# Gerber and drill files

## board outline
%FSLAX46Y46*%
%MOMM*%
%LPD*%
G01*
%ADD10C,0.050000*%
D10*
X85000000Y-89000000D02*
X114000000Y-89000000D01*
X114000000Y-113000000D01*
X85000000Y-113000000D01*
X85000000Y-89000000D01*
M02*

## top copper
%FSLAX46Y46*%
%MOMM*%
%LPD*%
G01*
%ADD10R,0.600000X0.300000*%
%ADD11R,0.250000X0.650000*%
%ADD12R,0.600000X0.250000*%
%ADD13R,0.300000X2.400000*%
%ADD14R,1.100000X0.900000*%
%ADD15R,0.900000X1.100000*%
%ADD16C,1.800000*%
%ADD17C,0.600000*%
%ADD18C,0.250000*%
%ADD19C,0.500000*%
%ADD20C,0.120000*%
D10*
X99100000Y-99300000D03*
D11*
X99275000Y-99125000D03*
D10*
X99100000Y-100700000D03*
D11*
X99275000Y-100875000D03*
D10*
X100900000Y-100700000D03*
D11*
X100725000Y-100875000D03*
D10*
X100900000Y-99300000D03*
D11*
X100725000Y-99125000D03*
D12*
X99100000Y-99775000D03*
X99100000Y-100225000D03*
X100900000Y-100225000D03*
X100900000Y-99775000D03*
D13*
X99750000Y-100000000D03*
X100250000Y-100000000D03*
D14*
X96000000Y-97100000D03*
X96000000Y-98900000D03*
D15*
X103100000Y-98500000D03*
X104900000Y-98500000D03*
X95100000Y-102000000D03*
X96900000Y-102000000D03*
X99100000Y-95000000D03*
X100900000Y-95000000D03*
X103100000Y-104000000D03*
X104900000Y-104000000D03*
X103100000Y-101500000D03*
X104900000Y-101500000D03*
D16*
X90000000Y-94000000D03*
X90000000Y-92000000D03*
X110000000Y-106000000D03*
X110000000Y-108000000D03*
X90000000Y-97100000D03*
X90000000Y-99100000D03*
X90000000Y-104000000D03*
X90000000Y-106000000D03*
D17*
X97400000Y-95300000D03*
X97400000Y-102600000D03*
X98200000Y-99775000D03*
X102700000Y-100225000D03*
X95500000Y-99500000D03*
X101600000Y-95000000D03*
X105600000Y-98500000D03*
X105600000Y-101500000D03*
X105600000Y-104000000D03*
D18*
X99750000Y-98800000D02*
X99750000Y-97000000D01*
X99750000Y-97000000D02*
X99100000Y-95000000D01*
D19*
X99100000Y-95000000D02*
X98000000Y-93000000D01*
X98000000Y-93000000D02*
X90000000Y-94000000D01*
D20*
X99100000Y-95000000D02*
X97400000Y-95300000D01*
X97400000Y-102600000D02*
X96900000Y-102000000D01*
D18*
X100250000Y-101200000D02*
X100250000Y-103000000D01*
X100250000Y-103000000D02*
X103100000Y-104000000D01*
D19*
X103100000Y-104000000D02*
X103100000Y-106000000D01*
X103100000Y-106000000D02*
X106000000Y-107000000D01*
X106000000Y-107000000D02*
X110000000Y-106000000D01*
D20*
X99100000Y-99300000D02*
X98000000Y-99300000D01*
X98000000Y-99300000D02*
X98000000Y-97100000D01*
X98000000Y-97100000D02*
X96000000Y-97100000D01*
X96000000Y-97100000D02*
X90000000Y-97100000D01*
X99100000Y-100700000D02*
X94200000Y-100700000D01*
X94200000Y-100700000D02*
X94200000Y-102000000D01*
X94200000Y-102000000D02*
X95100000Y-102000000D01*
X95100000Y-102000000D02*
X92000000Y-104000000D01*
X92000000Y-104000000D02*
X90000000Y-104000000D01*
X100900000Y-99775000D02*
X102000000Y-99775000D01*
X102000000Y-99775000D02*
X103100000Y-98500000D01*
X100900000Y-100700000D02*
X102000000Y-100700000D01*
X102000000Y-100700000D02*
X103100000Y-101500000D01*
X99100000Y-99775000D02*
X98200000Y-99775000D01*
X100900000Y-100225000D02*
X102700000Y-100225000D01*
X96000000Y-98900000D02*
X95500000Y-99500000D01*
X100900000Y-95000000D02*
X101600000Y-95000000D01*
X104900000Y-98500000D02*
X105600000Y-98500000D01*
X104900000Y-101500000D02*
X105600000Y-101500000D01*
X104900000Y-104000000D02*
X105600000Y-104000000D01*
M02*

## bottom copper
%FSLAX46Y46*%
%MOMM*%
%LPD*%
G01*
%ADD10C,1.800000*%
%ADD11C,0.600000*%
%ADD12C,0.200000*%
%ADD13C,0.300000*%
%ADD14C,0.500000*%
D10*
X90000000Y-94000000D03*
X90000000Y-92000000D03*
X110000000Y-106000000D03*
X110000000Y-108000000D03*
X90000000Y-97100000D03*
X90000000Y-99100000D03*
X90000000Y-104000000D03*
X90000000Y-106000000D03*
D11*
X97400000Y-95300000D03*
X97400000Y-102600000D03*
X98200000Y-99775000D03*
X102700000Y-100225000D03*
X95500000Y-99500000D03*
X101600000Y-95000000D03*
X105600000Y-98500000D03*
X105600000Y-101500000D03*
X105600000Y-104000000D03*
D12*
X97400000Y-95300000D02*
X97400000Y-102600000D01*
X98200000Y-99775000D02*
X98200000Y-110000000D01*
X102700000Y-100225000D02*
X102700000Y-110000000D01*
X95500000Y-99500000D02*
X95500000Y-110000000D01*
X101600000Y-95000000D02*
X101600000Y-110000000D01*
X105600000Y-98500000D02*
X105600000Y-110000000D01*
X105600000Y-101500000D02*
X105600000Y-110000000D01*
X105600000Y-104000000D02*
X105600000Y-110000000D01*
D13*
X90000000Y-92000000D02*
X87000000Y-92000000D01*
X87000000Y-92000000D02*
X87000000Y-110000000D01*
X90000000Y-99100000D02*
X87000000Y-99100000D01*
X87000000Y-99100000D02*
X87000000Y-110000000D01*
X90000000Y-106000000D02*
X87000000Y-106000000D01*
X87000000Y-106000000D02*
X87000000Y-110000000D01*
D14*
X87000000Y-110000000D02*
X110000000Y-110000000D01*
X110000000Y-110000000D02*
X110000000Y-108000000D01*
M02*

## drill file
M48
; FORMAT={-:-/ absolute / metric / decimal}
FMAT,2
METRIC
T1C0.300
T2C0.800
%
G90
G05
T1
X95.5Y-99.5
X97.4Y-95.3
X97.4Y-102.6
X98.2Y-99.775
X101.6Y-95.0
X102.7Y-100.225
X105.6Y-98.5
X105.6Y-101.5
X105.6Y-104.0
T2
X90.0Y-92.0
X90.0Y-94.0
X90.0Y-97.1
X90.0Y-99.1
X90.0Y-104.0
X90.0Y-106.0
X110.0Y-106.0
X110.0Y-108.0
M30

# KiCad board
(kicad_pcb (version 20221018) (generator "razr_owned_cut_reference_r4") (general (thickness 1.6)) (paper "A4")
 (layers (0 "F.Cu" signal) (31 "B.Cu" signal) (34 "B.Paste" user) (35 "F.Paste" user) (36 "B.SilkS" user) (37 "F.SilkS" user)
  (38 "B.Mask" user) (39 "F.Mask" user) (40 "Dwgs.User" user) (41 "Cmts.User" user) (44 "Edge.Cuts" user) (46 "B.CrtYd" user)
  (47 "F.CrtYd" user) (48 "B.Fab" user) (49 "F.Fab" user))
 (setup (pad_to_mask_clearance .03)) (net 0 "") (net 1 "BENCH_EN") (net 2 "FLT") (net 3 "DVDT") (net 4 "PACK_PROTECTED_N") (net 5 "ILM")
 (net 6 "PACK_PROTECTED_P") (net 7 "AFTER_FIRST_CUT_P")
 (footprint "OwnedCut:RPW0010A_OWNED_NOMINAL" (layer "F.Cu") (at 100 100)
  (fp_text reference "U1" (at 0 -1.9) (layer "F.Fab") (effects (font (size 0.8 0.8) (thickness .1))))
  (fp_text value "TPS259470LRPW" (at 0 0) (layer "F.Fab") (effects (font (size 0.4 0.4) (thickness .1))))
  (pad "1" smd rect (at -0.9 -0.7) (size 0.6 0.3) (layers "F.Cu" "F.Paste" "F.Mask") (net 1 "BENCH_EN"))
  (pad "1" smd rect (at -0.725 -0.875) (size 0.25 0.65) (layers "F.Cu" "F.Paste" "F.Mask") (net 1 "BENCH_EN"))
  (pad "4" smd rect (at -0.9 0.7) (size 0.6 0.3) (layers "F.Cu" "F.Paste" "F.Mask") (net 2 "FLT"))
  (pad "4" smd rect (at -0.725 0.875) (size 0.25 0.65) (layers "F.Cu" "F.Paste" "F.Mask") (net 2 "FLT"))
  (pad "7" smd rect (at 0.9 0.7) (size 0.6 0.3) (layers "F.Cu" "F.Paste" "F.Mask") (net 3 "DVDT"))
  (pad "7" smd rect (at 0.725 0.875) (size 0.25 0.65) (layers "F.Cu" "F.Paste" "F.Mask") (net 3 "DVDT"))
  (pad "10" smd rect (at 0.9 -0.7) (size 0.6 0.3) (layers "F.Cu" "F.Paste" "F.Mask"))
  (pad "10" smd rect (at 0.725 -0.875) (size 0.25 0.65) (layers "F.Cu" "F.Paste" "F.Mask"))
  (pad "2" smd rect (at -0.9 -0.225) (size 0.6 0.25) (layers "F.Cu" "F.Paste" "F.Mask") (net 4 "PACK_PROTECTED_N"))
  (pad "3" smd rect (at -0.9 0.225) (size 0.6 0.25) (layers "F.Cu" "F.Paste" "F.Mask"))
  (pad "8" smd rect (at 0.9 0.225) (size 0.6 0.25) (layers "F.Cu" "F.Paste" "F.Mask") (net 4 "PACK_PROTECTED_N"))
  (pad "9" smd rect (at 0.9 -0.225) (size 0.6 0.25) (layers "F.Cu" "F.Paste" "F.Mask") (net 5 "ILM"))
  (pad "5" smd rect (at -0.25 0) (size 0.3 2.4) (layers "F.Cu" "F.Paste" "F.Mask") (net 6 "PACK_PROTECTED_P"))
  (pad "6" smd rect (at 0.25 0) (size 0.3 2.4) (layers "F.Cu" "F.Paste" "F.Mask") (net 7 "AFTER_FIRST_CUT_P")))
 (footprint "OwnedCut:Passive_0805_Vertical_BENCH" (layer "F.Cu") (at 96 98)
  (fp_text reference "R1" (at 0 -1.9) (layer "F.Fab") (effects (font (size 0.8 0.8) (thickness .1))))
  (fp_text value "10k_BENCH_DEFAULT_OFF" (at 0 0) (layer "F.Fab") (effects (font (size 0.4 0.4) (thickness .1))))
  (pad "1" smd rect (at 0 -0.9) (size 1.1 0.9) (layers "F.Cu" "F.Paste" "F.Mask") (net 1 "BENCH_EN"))
  (pad "2" smd rect (at 0 0.9) (size 1.1 0.9) (layers "F.Cu" "F.Paste" "F.Mask") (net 4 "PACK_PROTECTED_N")))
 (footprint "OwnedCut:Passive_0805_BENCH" (layer "F.Cu") (at 104 98.5)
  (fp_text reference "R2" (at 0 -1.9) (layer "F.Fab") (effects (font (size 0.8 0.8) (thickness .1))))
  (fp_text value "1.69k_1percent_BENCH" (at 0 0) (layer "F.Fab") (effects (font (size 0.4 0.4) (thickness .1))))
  (pad "1" smd rect (at -0.9 0) (size 0.9 1.1) (layers "F.Cu" "F.Paste" "F.Mask") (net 5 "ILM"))
  (pad "2" smd rect (at 0.9 0) (size 0.9 1.1) (layers "F.Cu" "F.Paste" "F.Mask") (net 4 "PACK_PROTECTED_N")))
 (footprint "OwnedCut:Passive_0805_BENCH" (layer "F.Cu") (at 96 102)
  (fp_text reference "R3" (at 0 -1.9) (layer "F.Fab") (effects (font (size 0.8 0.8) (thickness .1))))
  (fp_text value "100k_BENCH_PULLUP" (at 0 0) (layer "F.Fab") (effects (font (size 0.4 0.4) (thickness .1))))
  (pad "1" smd rect (at -0.9 0) (size 0.9 1.1) (layers "F.Cu" "F.Paste" "F.Mask") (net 2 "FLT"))
  (pad "2" smd rect (at 0.9 0) (size 0.9 1.1) (layers "F.Cu" "F.Paste" "F.Mask") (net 6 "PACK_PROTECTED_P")))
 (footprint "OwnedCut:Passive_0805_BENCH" (layer "F.Cu") (at 100 95)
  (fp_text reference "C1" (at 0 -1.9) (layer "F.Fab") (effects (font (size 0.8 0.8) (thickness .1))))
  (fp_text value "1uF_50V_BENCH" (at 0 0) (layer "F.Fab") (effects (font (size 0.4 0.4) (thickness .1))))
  (pad "1" smd rect (at -0.9 0) (size 0.9 1.1) (layers "F.Cu" "F.Paste" "F.Mask") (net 6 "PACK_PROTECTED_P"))
  (pad "2" smd rect (at 0.9 0) (size 0.9 1.1) (layers "F.Cu" "F.Paste" "F.Mask") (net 4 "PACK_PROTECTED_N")))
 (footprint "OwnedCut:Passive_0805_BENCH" (layer "F.Cu") (at 104 104)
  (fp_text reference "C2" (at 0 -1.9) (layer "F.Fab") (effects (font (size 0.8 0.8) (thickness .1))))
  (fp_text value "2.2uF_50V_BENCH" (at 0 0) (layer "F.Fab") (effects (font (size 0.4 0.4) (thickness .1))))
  (pad "1" smd rect (at -0.9 0) (size 0.9 1.1) (layers "F.Cu" "F.Paste" "F.Mask") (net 7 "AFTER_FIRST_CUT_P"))
  (pad "2" smd rect (at 0.9 0) (size 0.9 1.1) (layers "F.Cu" "F.Paste" "F.Mask") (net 4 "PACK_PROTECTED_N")))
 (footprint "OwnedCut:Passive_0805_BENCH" (layer "F.Cu") (at 104 101.5)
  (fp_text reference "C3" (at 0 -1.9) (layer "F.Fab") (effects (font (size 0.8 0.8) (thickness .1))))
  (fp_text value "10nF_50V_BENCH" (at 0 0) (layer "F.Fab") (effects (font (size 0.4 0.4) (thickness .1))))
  (pad "1" smd rect (at -0.9 0) (size 0.9 1.1) (layers "F.Cu" "F.Paste" "F.Mask") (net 3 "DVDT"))
  (pad "2" smd rect (at 0.9 0) (size 0.9 1.1) (layers "F.Cu" "F.Paste" "F.Mask") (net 4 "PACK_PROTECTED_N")))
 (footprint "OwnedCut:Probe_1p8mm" (layer "F.Cu") (at 90 94)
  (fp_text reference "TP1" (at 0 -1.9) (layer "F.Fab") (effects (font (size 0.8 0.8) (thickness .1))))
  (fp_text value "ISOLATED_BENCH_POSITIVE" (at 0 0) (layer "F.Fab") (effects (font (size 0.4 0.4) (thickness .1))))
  (pad "1" thru_hole circle (at 0 0) (size 1.8 1.8) (drill .8) (layers "*.Cu" "*.Mask") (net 6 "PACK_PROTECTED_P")))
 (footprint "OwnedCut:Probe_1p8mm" (layer "F.Cu") (at 90 92)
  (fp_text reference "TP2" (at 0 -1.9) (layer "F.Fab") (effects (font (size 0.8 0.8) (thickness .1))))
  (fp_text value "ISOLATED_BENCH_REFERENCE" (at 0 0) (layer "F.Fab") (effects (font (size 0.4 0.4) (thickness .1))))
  (pad "1" thru_hole circle (at 0 0) (size 1.8 1.8) (drill .8) (layers "*.Cu" "*.Mask") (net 4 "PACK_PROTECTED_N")))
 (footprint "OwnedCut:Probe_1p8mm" (layer "F.Cu") (at 110 106)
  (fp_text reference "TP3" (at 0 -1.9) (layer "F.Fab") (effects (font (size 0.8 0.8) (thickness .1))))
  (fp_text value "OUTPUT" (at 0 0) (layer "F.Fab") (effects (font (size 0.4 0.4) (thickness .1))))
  (pad "1" thru_hole circle (at 0 0) (size 1.8 1.8) (drill .8) (layers "*.Cu" "*.Mask") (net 7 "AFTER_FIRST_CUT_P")))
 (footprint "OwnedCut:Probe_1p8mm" (layer "F.Cu") (at 110 108)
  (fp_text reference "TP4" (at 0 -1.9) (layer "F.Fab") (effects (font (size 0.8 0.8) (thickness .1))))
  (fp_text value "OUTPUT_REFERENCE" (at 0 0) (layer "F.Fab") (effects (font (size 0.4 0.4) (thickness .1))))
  (pad "1" thru_hole circle (at 0 0) (size 1.8 1.8) (drill .8) (layers "*.Cu" "*.Mask") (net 4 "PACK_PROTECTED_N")))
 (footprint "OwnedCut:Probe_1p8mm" (layer "F.Cu") (at 90 97.1)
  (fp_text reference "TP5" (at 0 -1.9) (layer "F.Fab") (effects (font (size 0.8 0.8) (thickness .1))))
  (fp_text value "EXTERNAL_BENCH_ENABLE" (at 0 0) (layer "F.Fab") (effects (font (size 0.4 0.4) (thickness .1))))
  (pad "1" thru_hole circle (at 0 0) (size 1.8 1.8) (drill .8) (layers "*.Cu" "*.Mask") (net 1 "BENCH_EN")))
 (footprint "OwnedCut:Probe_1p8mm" (layer "F.Cu") (at 90 99.1)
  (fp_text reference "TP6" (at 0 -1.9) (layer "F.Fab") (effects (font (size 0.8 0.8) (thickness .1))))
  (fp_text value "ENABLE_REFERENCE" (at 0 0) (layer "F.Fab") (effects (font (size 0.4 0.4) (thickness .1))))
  (pad "1" thru_hole circle (at 0 0) (size 1.8 1.8) (drill .8) (layers "*.Cu" "*.Mask") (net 4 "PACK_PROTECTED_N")))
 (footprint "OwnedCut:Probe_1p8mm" (layer "F.Cu") (at 90 104)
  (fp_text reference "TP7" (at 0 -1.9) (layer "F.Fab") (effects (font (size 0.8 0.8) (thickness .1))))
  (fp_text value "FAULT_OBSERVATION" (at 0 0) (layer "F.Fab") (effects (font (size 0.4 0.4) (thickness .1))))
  (pad "1" thru_hole circle (at 0 0) (size 1.8 1.8) (drill .8) (layers "*.Cu" "*.Mask") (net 2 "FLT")))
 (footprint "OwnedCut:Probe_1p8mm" (layer "F.Cu") (at 90 106)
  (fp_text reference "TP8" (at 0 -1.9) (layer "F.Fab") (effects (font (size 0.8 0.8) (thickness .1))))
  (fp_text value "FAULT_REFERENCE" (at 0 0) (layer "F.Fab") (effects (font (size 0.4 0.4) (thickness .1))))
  (pad "1" thru_hole circle (at 0 0) (size 1.8 1.8) (drill .8) (layers "*.Cu" "*.Mask") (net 4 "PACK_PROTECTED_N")))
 (segment (start 99.75 98.8) (end 99.75 97) (width 0.25) (layer "F.Cu") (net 6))
 (segment (start 99.75 97) (end 99.1 95) (width 0.25) (layer "F.Cu") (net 6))
 (segment (start 99.1 95) (end 98 93) (width 0.5) (layer "F.Cu") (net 6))
 (segment (start 98 93) (end 90 94) (width 0.5) (layer "F.Cu") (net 6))
 (segment (start 99.1 95) (end 97.4 95.3) (width 0.12) (layer "F.Cu") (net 6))
 (via (at 97.4 95.3) (size .6) (drill .3) (layers "F.Cu" "B.Cu") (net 6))
 (segment (start 97.4 95.3) (end 97.4 102.6) (width 0.2) (layer "B.Cu") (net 6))
 (via (at 97.4 102.6) (size .6) (drill .3) (layers "F.Cu" "B.Cu") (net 6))
 (segment (start 97.4 102.6) (end 96.9 102) (width 0.12) (layer "F.Cu") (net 6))
 (segment (start 100.25 101.2) (end 100.25 103) (width 0.25) (layer "F.Cu") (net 7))
 (segment (start 100.25 103) (end 103.1 104) (width 0.25) (layer "F.Cu") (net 7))
 (segment (start 103.1 104) (end 103.1 106) (width 0.5) (layer "F.Cu") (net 7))
 (segment (start 103.1 106) (end 106 107) (width 0.5) (layer "F.Cu") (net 7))
 (segment (start 106 107) (end 110 106) (width 0.5) (layer "F.Cu") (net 7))
 (segment (start 99.1 99.3) (end 98 99.3) (width 0.12) (layer "F.Cu") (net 1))
 (segment (start 98 99.3) (end 98 97.1) (width 0.12) (layer "F.Cu") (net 1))
 (segment (start 98 97.1) (end 96 97.1) (width 0.12) (layer "F.Cu") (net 1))
 (segment (start 96 97.1) (end 90 97.1) (width 0.12) (layer "F.Cu") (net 1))
 (segment (start 99.1 100.7) (end 94.2 100.7) (width 0.12) (layer "F.Cu") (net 2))
 (segment (start 94.2 100.7) (end 94.2 102) (width 0.12) (layer "F.Cu") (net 2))
 (segment (start 94.2 102) (end 95.1 102) (width 0.12) (layer "F.Cu") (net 2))
 (segment (start 95.1 102) (end 92 104) (width 0.12) (layer "F.Cu") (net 2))
 (segment (start 92 104) (end 90 104) (width 0.12) (layer "F.Cu") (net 2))
 (segment (start 100.9 99.775) (end 102 99.775) (width 0.12) (layer "F.Cu") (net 5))
 (segment (start 102 99.775) (end 103.1 98.5) (width 0.12) (layer "F.Cu") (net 5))
 (segment (start 100.9 100.7) (end 102 100.7) (width 0.12) (layer "F.Cu") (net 3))
 (segment (start 102 100.7) (end 103.1 101.5) (width 0.12) (layer "F.Cu") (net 3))
 (segment (start 99.1 99.775) (end 98.2 99.775) (width 0.12) (layer "F.Cu") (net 4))
 (via (at 98.2 99.775) (size .6) (drill .3) (layers "F.Cu" "B.Cu") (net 4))
 (segment (start 98.2 99.775) (end 98.2 110) (width 0.2) (layer "B.Cu") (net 4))
 (segment (start 100.9 100.225) (end 102.7 100.225) (width 0.12) (layer "F.Cu") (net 4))
 (via (at 102.7 100.225) (size .6) (drill .3) (layers "F.Cu" "B.Cu") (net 4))
 (segment (start 102.7 100.225) (end 102.7 110) (width 0.2) (layer "B.Cu") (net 4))
 (segment (start 96 98.9) (end 95.5 99.5) (width 0.12) (layer "F.Cu") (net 4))
 (via (at 95.5 99.5) (size .6) (drill .3) (layers "F.Cu" "B.Cu") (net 4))
 (segment (start 95.5 99.5) (end 95.5 110) (width 0.2) (layer "B.Cu") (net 4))
 (segment (start 100.9 95) (end 101.6 95) (width 0.12) (layer "F.Cu") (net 4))
 (via (at 101.6 95) (size .6) (drill .3) (layers "F.Cu" "B.Cu") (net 4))
 (segment (start 101.6 95) (end 101.6 110) (width 0.2) (layer "B.Cu") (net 4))
 (segment (start 104.9 98.5) (end 105.6 98.5) (width 0.12) (layer "F.Cu") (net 4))
 (via (at 105.6 98.5) (size .6) (drill .3) (layers "F.Cu" "B.Cu") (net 4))
 (segment (start 105.6 98.5) (end 105.6 110) (width 0.2) (layer "B.Cu") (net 4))
 (segment (start 104.9 101.5) (end 105.6 101.5) (width 0.12) (layer "F.Cu") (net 4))
 (via (at 105.6 101.5) (size .6) (drill .3) (layers "F.Cu" "B.Cu") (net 4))
 (segment (start 105.6 101.5) (end 105.6 110) (width 0.2) (layer "B.Cu") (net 4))
 (segment (start 104.9 104) (end 105.6 104) (width 0.12) (layer "F.Cu") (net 4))
 (via (at 105.6 104) (size .6) (drill .3) (layers "F.Cu" "B.Cu") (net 4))
 (segment (start 105.6 104) (end 105.6 110) (width 0.2) (layer "B.Cu") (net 4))
 (segment (start 90 92) (end 87 92) (width 0.3) (layer "B.Cu") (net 4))
 (segment (start 87 92) (end 87 110) (width 0.3) (layer "B.Cu") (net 4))
 (segment (start 90 99.1) (end 87 99.1) (width 0.3) (layer "B.Cu") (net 4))
 (segment (start 87 99.1) (end 87 110) (width 0.3) (layer "B.Cu") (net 4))
 (segment (start 90 106) (end 87 106) (width 0.3) (layer "B.Cu") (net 4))
 (segment (start 87 106) (end 87 110) (width 0.3) (layer "B.Cu") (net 4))
 (segment (start 87 110) (end 110 110) (width 0.5) (layer "B.Cu") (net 4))
 (segment (start 110 110) (end 110 108) (width 0.5) (layer "B.Cu") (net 4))
 (gr_rect (start 85 89) (end 114 113) (stroke (width .05) (type default)) (fill none) (layer "Edge.Cuts")))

